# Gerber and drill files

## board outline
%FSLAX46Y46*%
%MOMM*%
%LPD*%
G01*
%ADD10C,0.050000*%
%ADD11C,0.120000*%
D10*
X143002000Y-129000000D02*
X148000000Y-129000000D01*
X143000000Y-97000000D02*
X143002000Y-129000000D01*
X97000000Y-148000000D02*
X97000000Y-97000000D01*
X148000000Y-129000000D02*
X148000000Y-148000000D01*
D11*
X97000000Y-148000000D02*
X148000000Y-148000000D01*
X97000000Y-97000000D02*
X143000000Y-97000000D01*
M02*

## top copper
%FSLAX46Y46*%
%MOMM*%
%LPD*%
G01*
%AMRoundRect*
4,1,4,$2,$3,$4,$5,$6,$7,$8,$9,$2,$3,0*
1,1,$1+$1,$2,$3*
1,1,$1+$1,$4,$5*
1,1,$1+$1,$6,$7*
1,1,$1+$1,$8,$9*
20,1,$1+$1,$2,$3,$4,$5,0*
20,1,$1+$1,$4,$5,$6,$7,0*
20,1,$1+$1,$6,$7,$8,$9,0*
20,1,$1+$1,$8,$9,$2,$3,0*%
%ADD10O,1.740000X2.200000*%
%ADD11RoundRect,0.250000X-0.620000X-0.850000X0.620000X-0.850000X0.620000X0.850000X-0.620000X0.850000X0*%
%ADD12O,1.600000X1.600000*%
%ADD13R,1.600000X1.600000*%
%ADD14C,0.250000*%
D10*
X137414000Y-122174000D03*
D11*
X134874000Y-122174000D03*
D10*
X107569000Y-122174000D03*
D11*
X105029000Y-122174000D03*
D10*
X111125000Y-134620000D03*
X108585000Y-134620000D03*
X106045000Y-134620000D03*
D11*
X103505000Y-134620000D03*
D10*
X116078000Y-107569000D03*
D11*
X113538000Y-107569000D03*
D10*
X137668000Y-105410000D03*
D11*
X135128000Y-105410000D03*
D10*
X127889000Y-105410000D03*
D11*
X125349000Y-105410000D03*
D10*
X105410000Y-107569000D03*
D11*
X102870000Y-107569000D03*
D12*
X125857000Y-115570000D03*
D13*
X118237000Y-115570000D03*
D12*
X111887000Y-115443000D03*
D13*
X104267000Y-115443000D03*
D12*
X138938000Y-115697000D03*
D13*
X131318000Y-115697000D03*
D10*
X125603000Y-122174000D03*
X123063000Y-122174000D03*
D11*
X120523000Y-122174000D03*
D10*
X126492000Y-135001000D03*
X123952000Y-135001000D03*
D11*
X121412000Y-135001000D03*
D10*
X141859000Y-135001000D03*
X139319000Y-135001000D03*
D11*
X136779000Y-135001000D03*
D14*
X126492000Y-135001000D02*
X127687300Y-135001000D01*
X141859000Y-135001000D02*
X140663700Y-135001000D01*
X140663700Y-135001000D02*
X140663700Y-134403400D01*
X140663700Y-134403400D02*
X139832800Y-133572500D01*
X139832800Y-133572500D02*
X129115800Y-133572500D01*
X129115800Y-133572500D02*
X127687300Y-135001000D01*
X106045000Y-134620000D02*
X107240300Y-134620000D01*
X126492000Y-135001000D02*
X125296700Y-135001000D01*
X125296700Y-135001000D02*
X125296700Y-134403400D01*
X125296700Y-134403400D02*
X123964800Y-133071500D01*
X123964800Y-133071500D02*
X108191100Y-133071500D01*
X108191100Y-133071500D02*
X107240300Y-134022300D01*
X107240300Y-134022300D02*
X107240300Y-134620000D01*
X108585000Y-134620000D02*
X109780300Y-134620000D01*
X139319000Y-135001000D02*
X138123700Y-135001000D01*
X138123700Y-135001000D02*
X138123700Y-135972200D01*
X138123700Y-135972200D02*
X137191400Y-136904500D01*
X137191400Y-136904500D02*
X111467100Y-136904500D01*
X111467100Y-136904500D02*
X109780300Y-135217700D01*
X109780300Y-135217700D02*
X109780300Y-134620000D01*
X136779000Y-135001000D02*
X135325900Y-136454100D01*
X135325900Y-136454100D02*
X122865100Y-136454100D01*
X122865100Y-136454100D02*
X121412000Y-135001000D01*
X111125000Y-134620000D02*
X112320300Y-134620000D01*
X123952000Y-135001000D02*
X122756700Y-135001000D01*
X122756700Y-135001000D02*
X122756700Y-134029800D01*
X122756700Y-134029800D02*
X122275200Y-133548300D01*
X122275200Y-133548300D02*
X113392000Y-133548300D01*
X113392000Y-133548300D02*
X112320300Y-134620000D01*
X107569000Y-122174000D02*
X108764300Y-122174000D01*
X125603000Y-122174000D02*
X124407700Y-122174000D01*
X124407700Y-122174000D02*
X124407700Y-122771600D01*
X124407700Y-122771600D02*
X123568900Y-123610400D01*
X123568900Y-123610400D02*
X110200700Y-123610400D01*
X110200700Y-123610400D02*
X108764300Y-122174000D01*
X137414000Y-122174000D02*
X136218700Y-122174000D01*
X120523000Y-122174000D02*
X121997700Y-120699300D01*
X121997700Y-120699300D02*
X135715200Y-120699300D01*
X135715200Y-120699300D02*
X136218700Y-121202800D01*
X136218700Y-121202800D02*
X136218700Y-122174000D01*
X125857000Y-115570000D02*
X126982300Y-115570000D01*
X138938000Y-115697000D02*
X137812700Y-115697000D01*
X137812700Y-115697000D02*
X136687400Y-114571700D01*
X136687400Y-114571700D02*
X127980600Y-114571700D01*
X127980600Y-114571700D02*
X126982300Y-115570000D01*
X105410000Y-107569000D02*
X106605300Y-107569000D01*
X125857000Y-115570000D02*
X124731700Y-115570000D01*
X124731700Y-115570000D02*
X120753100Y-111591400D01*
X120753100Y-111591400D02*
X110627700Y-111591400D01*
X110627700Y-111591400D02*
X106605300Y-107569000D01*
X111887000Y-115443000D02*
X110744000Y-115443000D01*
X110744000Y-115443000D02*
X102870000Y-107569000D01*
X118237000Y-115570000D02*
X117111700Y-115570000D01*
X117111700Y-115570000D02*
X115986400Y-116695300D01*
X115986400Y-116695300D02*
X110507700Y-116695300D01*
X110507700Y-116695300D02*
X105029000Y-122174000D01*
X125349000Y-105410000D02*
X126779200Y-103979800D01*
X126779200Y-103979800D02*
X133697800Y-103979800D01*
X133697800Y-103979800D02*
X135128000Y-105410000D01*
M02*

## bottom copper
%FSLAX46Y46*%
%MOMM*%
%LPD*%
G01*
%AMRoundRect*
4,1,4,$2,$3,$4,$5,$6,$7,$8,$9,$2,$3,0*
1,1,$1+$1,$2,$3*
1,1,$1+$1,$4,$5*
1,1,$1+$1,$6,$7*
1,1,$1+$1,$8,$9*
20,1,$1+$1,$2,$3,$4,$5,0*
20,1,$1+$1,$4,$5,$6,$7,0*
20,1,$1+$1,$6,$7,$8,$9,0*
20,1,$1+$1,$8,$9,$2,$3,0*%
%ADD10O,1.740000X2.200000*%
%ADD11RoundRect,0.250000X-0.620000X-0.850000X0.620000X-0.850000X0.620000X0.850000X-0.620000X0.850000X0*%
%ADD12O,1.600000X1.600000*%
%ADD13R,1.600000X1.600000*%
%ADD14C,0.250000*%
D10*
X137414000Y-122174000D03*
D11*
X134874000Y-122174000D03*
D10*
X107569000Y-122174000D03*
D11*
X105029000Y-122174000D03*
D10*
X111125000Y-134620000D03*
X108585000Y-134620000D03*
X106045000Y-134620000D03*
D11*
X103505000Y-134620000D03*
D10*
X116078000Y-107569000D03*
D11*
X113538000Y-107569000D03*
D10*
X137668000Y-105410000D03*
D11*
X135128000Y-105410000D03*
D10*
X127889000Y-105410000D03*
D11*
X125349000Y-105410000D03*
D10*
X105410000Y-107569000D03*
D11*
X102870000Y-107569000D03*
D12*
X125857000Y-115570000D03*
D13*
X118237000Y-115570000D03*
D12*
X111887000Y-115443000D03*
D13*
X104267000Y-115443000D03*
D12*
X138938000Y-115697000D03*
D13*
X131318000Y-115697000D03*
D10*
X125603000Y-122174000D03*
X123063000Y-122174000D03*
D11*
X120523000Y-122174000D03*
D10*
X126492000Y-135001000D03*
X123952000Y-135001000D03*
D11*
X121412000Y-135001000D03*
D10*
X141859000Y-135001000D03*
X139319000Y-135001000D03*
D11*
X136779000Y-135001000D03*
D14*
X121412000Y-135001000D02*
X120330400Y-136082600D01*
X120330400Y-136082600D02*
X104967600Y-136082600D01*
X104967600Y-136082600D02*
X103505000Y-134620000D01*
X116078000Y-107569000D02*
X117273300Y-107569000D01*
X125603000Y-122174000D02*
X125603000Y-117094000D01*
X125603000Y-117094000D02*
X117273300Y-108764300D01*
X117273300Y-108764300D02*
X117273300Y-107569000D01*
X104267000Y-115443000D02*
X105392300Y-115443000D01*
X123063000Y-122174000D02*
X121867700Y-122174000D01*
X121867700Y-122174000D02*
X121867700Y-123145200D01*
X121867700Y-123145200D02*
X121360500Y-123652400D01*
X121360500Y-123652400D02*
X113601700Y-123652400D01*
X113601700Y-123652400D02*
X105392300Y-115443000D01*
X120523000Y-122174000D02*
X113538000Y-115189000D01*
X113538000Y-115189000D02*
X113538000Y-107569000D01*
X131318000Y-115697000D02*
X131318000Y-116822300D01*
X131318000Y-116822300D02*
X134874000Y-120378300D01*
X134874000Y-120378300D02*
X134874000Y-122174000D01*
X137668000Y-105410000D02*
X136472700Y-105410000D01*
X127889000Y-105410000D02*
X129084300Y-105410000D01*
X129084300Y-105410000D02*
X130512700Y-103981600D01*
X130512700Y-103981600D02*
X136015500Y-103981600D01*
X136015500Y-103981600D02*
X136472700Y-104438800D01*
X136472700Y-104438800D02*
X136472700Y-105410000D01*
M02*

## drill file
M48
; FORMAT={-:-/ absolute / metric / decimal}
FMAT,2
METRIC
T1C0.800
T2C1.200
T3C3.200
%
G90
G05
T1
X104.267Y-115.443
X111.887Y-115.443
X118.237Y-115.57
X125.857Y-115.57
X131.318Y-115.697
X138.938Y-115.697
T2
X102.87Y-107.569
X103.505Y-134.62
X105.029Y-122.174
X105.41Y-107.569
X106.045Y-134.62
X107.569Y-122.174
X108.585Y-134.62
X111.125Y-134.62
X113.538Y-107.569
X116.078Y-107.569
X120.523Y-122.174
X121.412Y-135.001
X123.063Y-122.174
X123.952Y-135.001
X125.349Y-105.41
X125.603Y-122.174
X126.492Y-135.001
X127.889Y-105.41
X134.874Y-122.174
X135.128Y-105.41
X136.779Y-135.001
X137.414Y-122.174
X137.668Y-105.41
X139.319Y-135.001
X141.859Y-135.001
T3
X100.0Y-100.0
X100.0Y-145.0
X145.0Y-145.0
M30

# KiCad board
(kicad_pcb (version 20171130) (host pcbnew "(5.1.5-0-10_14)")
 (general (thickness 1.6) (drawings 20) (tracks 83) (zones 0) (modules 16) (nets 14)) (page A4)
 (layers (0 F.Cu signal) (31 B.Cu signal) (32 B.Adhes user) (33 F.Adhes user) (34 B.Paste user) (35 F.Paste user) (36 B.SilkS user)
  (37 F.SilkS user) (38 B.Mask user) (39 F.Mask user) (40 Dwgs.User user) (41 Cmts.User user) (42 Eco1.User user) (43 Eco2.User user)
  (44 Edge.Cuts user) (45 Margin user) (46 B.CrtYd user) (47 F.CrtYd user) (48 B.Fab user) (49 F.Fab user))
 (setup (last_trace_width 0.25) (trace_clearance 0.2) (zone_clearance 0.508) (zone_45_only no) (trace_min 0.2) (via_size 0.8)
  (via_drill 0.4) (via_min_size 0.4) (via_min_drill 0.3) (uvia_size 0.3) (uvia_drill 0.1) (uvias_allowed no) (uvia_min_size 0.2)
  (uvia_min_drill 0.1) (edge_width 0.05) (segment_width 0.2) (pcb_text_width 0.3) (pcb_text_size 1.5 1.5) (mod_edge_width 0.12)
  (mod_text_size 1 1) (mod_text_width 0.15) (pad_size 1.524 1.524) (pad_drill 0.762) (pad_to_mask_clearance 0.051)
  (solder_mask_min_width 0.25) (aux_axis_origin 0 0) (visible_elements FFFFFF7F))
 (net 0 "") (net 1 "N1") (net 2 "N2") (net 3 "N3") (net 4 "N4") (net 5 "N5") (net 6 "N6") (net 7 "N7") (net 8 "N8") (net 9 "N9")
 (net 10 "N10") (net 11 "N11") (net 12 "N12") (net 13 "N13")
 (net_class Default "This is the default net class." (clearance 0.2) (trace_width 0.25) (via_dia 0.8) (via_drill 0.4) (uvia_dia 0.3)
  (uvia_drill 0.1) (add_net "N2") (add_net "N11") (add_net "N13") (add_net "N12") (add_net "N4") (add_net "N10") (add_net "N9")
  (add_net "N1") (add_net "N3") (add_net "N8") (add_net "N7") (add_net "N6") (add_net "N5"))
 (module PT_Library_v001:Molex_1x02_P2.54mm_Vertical (layer F.Cu) (at 134.874 122.174)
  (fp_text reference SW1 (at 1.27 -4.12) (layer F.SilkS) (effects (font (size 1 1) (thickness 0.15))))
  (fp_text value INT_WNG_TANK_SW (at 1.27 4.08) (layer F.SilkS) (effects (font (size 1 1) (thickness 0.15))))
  (pad 2 thru_hole oval (at 2.54 0) (size 1.74 2.2) (drill 1.2) (layers *.Cu *.Mask) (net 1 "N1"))
  (pad 1 thru_hole roundrect (at 0 0) (size 1.74 2.2) (drill 1.2) (layers *.Cu *.Mask) (roundrect_rratio 0.143678) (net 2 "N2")))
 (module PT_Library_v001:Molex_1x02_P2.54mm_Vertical (layer F.Cu) (at 105.029 122.174)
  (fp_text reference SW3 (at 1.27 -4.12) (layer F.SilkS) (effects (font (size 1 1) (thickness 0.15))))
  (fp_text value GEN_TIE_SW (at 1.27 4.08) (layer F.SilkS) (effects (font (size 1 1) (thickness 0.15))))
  (pad 2 thru_hole oval (at 2.54 0) (size 1.74 2.2) (drill 1.2) (layers *.Cu *.Mask) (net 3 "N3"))
  (pad 1 thru_hole roundrect (at 0 0) (size 1.74 2.2) (drill 1.2) (layers *.Cu *.Mask) (roundrect_rratio 0.143678) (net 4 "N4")))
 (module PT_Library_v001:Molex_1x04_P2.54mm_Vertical (layer F.Cu) (at 103.505 134.62)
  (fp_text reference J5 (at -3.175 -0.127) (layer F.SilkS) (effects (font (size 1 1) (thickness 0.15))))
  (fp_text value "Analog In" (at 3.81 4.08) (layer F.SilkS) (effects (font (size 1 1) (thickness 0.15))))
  (pad 4 thru_hole oval (at 7.62 0) (size 1.74 2.2) (drill 1.2) (layers *.Cu *.Mask) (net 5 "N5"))
  (pad 3 thru_hole oval (at 5.08 0) (size 1.74 2.2) (drill 1.2) (layers *.Cu *.Mask) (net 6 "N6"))
  (pad 2 thru_hole oval (at 2.54 0) (size 1.74 2.2) (drill 1.2) (layers *.Cu *.Mask) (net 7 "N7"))
  (pad 1 thru_hole roundrect (at 0 0) (size 1.74 2.2) (drill 1.2) (layers *.Cu *.Mask) (roundrect_rratio 0.143678) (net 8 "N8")))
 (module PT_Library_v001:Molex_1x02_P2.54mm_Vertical (layer F.Cu) (at 113.538 107.569)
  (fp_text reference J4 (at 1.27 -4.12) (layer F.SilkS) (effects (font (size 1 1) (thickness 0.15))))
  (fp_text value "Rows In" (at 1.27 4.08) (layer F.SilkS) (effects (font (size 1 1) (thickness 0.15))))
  (pad 2 thru_hole oval (at 2.54 0) (size 1.74 2.2) (drill 1.2) (layers *.Cu *.Mask) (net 3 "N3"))
  (pad 1 thru_hole roundrect (at 0 0) (size 1.74 2.2) (drill 1.2) (layers *.Cu *.Mask) (roundrect_rratio 0.143678) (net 1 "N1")))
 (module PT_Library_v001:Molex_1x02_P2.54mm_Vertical (layer F.Cu) (at 135.128 105.41)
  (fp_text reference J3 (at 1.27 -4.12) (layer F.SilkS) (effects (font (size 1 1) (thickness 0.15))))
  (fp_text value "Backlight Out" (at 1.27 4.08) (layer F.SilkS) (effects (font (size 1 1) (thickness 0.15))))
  (pad 2 thru_hole oval (at 2.54 0) (size 1.74 2.2) (drill 1.2) (layers *.Cu *.Mask) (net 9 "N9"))
  (pad 1 thru_hole roundrect (at 0 0) (size 1.74 2.2) (drill 1.2) (layers *.Cu *.Mask) (roundrect_rratio 0.143678) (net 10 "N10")))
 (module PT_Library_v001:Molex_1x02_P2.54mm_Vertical (layer F.Cu) (at 125.349 105.41)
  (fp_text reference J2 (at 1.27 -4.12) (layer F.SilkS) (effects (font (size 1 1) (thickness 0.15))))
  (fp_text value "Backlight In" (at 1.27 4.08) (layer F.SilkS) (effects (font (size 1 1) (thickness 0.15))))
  (pad 2 thru_hole oval (at 2.54 0) (size 1.74 2.2) (drill 1.2) (layers *.Cu *.Mask) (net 9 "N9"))
  (pad 1 thru_hole roundrect (at 0 0) (size 1.74 2.2) (drill 1.2) (layers *.Cu *.Mask) (roundrect_rratio 0.143678) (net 10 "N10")))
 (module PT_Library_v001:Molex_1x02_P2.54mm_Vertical (layer F.Cu) (at 102.87 107.569)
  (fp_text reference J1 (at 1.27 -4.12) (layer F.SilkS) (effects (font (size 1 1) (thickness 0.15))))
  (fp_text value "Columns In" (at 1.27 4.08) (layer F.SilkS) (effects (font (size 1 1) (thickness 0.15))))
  (pad 2 thru_hole oval (at 2.54 0) (size 1.74 2.2) (drill 1.2) (layers *.Cu *.Mask) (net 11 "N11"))
  (pad 1 thru_hole roundrect (at 0 0) (size 1.74 2.2) (drill 1.2) (layers *.Cu *.Mask) (roundrect_rratio 0.143678) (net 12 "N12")))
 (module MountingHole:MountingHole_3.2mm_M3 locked (layer F.Cu) (at 145 145)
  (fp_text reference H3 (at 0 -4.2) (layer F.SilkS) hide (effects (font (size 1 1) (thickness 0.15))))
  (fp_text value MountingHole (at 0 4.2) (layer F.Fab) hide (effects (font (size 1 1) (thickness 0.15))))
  (pad 1 np_thru_hole circle (at 0 0) (size 3.2 3.2) (drill 3.2) (layers *.Cu *.Mask)))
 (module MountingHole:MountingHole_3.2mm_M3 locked (layer F.Cu) (at 100 100)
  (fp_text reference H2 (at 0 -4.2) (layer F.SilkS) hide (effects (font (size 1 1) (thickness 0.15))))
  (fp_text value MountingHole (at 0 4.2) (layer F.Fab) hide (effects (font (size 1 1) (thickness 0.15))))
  (pad 1 np_thru_hole circle (at 0 0) (size 3.2 3.2) (drill 3.2) (layers *.Cu *.Mask)))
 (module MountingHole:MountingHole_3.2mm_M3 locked (layer F.Cu) (at 100 145)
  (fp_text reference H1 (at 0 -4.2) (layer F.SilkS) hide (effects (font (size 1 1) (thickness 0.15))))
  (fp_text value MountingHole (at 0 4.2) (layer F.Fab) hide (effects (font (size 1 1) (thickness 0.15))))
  (pad 1 np_thru_hole circle (at 0 0) (size 3.2 3.2) (drill 3.2) (layers *.Cu *.Mask)))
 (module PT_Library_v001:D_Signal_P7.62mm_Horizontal (layer F.Cu) (at 118.237 115.57)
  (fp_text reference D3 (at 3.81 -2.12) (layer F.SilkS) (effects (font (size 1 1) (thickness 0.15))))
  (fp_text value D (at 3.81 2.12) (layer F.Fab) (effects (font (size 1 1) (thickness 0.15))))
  (pad 2 thru_hole oval (at 7.62 0) (size 1.6 1.6) (drill 0.8) (layers *.Cu *.Mask) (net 11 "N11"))
  (pad 1 thru_hole rect (at 0 0) (size 1.6 1.6) (drill 0.8) (layers *.Cu *.Mask) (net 4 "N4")))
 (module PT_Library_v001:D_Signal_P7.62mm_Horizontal (layer F.Cu) (at 104.267 115.443)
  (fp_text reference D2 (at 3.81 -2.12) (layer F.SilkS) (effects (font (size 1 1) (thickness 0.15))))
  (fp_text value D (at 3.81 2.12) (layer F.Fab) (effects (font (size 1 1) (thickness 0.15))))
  (pad 2 thru_hole oval (at 7.62 0) (size 1.6 1.6) (drill 0.8) (layers *.Cu *.Mask) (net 12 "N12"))
  (pad 1 thru_hole rect (at 0 0) (size 1.6 1.6) (drill 0.8) (layers *.Cu *.Mask) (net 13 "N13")))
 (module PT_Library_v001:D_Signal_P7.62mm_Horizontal (layer F.Cu) (at 131.318 115.697)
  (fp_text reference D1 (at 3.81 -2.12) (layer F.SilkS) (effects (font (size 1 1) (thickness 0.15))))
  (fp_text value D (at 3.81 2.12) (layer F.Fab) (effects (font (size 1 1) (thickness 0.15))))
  (pad 2 thru_hole oval (at 7.62 0) (size 1.6 1.6) (drill 0.8) (layers *.Cu *.Mask) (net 11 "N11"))
  (pad 1 thru_hole rect (at 0 0) (size 1.6 1.6) (drill 0.8) (layers *.Cu *.Mask) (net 2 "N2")))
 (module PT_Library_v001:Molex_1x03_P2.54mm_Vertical (layer F.Cu) (at 120.523 122.174)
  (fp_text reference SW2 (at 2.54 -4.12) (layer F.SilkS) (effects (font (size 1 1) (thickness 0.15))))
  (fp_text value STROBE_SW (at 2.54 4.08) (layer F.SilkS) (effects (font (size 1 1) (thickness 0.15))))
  (pad 3 thru_hole oval (at 5.08 0) (size 1.74 2.2) (drill 1.2) (layers *.Cu *.Mask) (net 3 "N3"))
  (pad 2 thru_hole oval (at 2.54 0) (size 1.74 2.2) (drill 1.2) (layers *.Cu *.Mask) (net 13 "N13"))
  (pad 1 thru_hole roundrect (at 0 0) (size 1.74 2.2) (drill 1.2) (layers *.Cu *.Mask) (roundrect_rratio 0.143678) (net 1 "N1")))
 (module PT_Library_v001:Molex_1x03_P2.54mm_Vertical (layer F.Cu) (at 121.412 135.001)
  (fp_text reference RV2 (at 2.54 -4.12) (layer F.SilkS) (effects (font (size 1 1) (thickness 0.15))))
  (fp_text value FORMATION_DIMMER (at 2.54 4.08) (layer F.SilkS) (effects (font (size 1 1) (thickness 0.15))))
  (pad 3 thru_hole oval (at 5.08 0) (size 1.74 2.2) (drill 1.2) (layers *.Cu *.Mask) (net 7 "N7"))
  (pad 2 thru_hole oval (at 2.54 0) (size 1.74 2.2) (drill 1.2) (layers *.Cu *.Mask) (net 5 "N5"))
  (pad 1 thru_hole roundrect (at 0 0) (size 1.74 2.2) (drill 1.2) (layers *.Cu *.Mask) (roundrect_rratio 0.143678) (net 8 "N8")))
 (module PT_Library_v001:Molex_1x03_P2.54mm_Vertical (layer F.Cu) (at 136.779 135.001)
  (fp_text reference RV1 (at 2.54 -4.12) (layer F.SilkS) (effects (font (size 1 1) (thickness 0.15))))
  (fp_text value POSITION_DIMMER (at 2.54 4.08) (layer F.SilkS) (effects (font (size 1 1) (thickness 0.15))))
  (pad 3 thru_hole oval (at 5.08 0) (size 1.74 2.2) (drill 1.2) (layers *.Cu *.Mask) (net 7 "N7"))
  (pad 2 thru_hole oval (at 2.54 0) (size 1.74 2.2) (drill 1.2) (layers *.Cu *.Mask) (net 6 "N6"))
  (pad 1 thru_hole roundrect (at 0 0) (size 1.74 2.2) (drill 1.2) (layers *.Cu *.Mask) (roundrect_rratio 0.143678) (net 8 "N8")))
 (gr_line (start 143.002 129) (end 148 129) (layer Edge.Cuts) (width 0.05))
 (gr_line (start 143 97) (end 143.002 129) (layer Edge.Cuts) (width 0.05))
 (gr_line (start 97 148) (end 97 97) (layer Edge.Cuts) (width 0.05))
 (gr_line (start 148 129) (end 148 148) (layer Edge.Cuts) (width 0.05))
 (gr_line (start 97 148) (end 148 148) (layer Edge.Cuts) (width 0.12))
 (gr_line (start 97 97) (end 143 97) (layer Edge.Cuts) (width 0.12))
 (segment (start 126.492 135.001) (end 127.6873 135.001) (width 0.25) (layer F.Cu) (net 7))
 (segment (start 141.859 135.001) (end 140.6637 135.001) (width 0.25) (layer F.Cu) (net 7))
 (segment (start 140.6637 135.001) (end 140.6637 134.4034) (width 0.25) (layer F.Cu) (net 7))
 (segment (start 140.6637 134.4034) (end 139.8328 133.5725) (width 0.25) (layer F.Cu) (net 7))
 (segment (start 139.8328 133.5725) (end 129.1158 133.5725) (width 0.25) (layer F.Cu) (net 7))
 (segment (start 129.1158 133.5725) (end 127.6873 135.001) (width 0.25) (layer F.Cu) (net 7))
 (segment (start 106.045 134.62) (end 107.2403 134.62) (width 0.25) (layer F.Cu) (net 7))
 (segment (start 126.492 135.001) (end 125.2967 135.001) (width 0.25) (layer F.Cu) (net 7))
 (segment (start 125.2967 135.001) (end 125.2967 134.4034) (width 0.25) (layer F.Cu) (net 7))
 (segment (start 125.2967 134.4034) (end 123.9648 133.0715) (width 0.25) (layer F.Cu) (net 7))
 (segment (start 123.9648 133.0715) (end 108.1911 133.0715) (width 0.25) (layer F.Cu) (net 7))
 (segment (start 108.1911 133.0715) (end 107.2403 134.0223) (width 0.25) (layer F.Cu) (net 7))
 (segment (start 107.2403 134.0223) (end 107.2403 134.62) (width 0.25) (layer F.Cu) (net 7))
 (segment (start 108.585 134.62) (end 109.7803 134.62) (width 0.25) (layer F.Cu) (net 6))
 (segment (start 139.319 135.001) (end 138.1237 135.001) (width 0.25) (layer F.Cu) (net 6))
 (segment (start 138.1237 135.001) (end 138.1237 135.9722) (width 0.25) (layer F.Cu) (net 6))
 (segment (start 138.1237 135.9722) (end 137.1914 136.9045) (width 0.25) (layer F.Cu) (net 6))
 (segment (start 137.1914 136.9045) (end 111.4671 136.9045) (width 0.25) (layer F.Cu) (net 6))
 (segment (start 111.4671 136.9045) (end 109.7803 135.2177) (width 0.25) (layer F.Cu) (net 6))
 (segment (start 109.7803 135.2177) (end 109.7803 134.62) (width 0.25) (layer F.Cu) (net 6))
 (segment (start 121.412 135.001) (end 120.3304 136.0826) (width 0.25) (layer B.Cu) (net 8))
 (segment (start 120.3304 136.0826) (end 104.9676 136.0826) (width 0.25) (layer B.Cu) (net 8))
 (segment (start 104.9676 136.0826) (end 103.505 134.62) (width 0.25) (layer B.Cu) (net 8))
 (segment (start 136.779 135.001) (end 135.3259 136.4541) (width 0.25) (layer F.Cu) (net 8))
 (segment (start 135.3259 136.4541) (end 122.8651 136.4541) (width 0.25) (layer F.Cu) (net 8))
 (segment (start 122.8651 136.4541) (end 121.412 135.001) (width 0.25) (layer F.Cu) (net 8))
 (segment (start 111.125 134.62) (end 112.3203 134.62) (width 0.25) (layer F.Cu) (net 5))
 (segment (start 123.952 135.001) (end 122.7567 135.001) (width 0.25) (layer F.Cu) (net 5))
 (segment (start 122.7567 135.001) (end 122.7567 134.0298) (width 0.25) (layer F.Cu) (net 5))
 (segment (start 122.7567 134.0298) (end 122.2752 133.5483) (width 0.25) (layer F.Cu) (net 5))
 (segment (start 122.2752 133.5483) (end 113.392 133.5483) (width 0.25) (layer F.Cu) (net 5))
 (segment (start 113.392 133.5483) (end 112.3203 134.62) (width 0.25) (layer F.Cu) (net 5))
 (segment (start 116.078 107.569) (end 117.2733 107.569) (width 0.25) (layer B.Cu) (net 3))
 (segment (start 125.603 122.174) (end 125.603 117.094) (width 0.25) (layer B.Cu) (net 3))
 (segment (start 125.603 117.094) (end 117.2733 108.7643) (width 0.25) (layer B.Cu) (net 3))
 (segment (start 117.2733 108.7643) (end 117.2733 107.569) (width 0.25) (layer B.Cu) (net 3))
 (segment (start 107.569 122.174) (end 108.7643 122.174) (width 0.25) (layer F.Cu) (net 3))
 (segment (start 125.603 122.174) (end 124.4077 122.174) (width 0.25) (layer F.Cu) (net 3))
 (segment (start 124.4077 122.174) (end 124.4077 122.7716) (width 0.25) (layer F.Cu) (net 3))
 (segment (start 124.4077 122.7716) (end 123.5689 123.6104) (width 0.25) (layer F.Cu) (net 3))
 (segment (start 123.5689 123.6104) (end 110.2007 123.6104) (width 0.25) (layer F.Cu) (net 3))
 (segment (start 110.2007 123.6104) (end 108.7643 122.174) (width 0.25) (layer F.Cu) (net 3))
 (segment (start 104.267 115.443) (end 105.3923 115.443) (width 0.25) (layer B.Cu) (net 13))
 (segment (start 123.063 122.174) (end 121.8677 122.174) (width 0.25) (layer B.Cu) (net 13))
 (segment (start 121.8677 122.174) (end 121.8677 123.1452) (width 0.25) (layer B.Cu) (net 13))
 (segment (start 121.8677 123.1452) (end 121.3605 123.6524) (width 0.25) (layer B.Cu) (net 13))
 (segment (start 121.3605 123.6524) (end 113.6017 123.6524) (width 0.25) (layer B.Cu) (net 13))
 (segment (start 113.6017 123.6524) (end 105.3923 115.443) (width 0.25) (layer B.Cu) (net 13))
 (segment (start 137.414 122.174) (end 136.2187 122.174) (width 0.25) (layer F.Cu) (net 1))
 (segment (start 120.523 122.174) (end 121.9977 120.6993) (width 0.25) (layer F.Cu) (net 1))
 (segment (start 121.9977 120.6993) (end 135.7152 120.6993) (width 0.25) (layer F.Cu) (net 1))
 (segment (start 135.7152 120.6993) (end 136.2187 121.2028) (width 0.25) (layer F.Cu) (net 1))
 (segment (start 136.2187 121.2028) (end 136.2187 122.174) (width 0.25) (layer F.Cu) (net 1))
 (segment (start 120.523 122.174) (end 113.538 115.189) (width 0.25) (layer B.Cu) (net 1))
 (segment (start 113.538 115.189) (end 113.538 107.569) (width 0.25) (layer B.Cu) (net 1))
 (segment (start 125.857 115.57) (end 126.9823 115.57) (width 0.25) (layer F.Cu) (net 11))
 (segment (start 138.938 115.697) (end 137.8127 115.697) (width 0.25) (layer F.Cu) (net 11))
 (segment (start 137.8127 115.697) (end 136.6874 114.5717) (width 0.25) (layer F.Cu) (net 11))
 (segment (start 136.6874 114.5717) (end 127.9806 114.5717) (width 0.25) (layer F.Cu) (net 11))
 (segment (start 127.9806 114.5717) (end 126.9823 115.57) (width 0.25) (layer F.Cu) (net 11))
 (segment (start 105.41 107.569) (end 106.6053 107.569) (width 0.25) (layer F.Cu) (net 11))
 (segment (start 125.857 115.57) (end 124.7317 115.57) (width 0.25) (layer F.Cu) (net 11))
 (segment (start 124.7317 115.57) (end 120.7531 111.5914) (width 0.25) (layer F.Cu) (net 11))
 (segment (start 120.7531 111.5914) (end 110.6277 111.5914) (width 0.25) (layer F.Cu) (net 11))
 (segment (start 110.6277 111.5914) (end 106.6053 107.569) (width 0.25) (layer F.Cu) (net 11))
 (segment (start 131.318 115.697) (end 131.318 116.8223) (width 0.25) (layer B.Cu) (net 2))
 (segment (start 131.318 116.8223) (end 134.874 120.3783) (width 0.25) (layer B.Cu) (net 2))
 (segment (start 134.874 120.3783) (end 134.874 122.174) (width 0.25) (layer B.Cu) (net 2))
 (segment (start 111.887 115.443) (end 110.744 115.443) (width 0.25) (layer F.Cu) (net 12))
 (segment (start 110.744 115.443) (end 102.87 107.569) (width 0.25) (layer F.Cu) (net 12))
 (segment (start 118.237 115.57) (end 117.1117 115.57) (width 0.25) (layer F.Cu) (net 4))
 (segment (start 117.1117 115.57) (end 115.9864 116.6953) (width 0.25) (layer F.Cu) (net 4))
 (segment (start 115.9864 116.6953) (end 110.5077 116.6953) (width 0.25) (layer F.Cu) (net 4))
 (segment (start 110.5077 116.6953) (end 105.029 122.174) (width 0.25) (layer F.Cu) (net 4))
 (segment (start 137.668 105.41) (end 136.4727 105.41) (width 0.25) (layer B.Cu) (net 9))
 (segment (start 127.889 105.41) (end 129.0843 105.41) (width 0.25) (layer B.Cu) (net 9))
 (segment (start 129.0843 105.41) (end 130.5127 103.9816) (width 0.25) (layer B.Cu) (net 9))
 (segment (start 130.5127 103.9816) (end 136.0155 103.9816) (width 0.25) (layer B.Cu) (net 9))
 (segment (start 136.0155 103.9816) (end 136.4727 104.4388) (width 0.25) (layer B.Cu) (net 9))
 (segment (start 136.4727 104.4388) (end 136.4727 105.41) (width 0.25) (layer B.Cu) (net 9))
 (segment (start 125.349 105.41) (end 126.7792 103.9798) (width 0.25) (layer F.Cu) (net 10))
 (segment (start 126.7792 103.9798) (end 133.6978 103.9798) (width 0.25) (layer F.Cu) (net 10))
 (segment (start 133.6978 103.9798) (end 135.128 105.41) (width 0.25) (layer F.Cu) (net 10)))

